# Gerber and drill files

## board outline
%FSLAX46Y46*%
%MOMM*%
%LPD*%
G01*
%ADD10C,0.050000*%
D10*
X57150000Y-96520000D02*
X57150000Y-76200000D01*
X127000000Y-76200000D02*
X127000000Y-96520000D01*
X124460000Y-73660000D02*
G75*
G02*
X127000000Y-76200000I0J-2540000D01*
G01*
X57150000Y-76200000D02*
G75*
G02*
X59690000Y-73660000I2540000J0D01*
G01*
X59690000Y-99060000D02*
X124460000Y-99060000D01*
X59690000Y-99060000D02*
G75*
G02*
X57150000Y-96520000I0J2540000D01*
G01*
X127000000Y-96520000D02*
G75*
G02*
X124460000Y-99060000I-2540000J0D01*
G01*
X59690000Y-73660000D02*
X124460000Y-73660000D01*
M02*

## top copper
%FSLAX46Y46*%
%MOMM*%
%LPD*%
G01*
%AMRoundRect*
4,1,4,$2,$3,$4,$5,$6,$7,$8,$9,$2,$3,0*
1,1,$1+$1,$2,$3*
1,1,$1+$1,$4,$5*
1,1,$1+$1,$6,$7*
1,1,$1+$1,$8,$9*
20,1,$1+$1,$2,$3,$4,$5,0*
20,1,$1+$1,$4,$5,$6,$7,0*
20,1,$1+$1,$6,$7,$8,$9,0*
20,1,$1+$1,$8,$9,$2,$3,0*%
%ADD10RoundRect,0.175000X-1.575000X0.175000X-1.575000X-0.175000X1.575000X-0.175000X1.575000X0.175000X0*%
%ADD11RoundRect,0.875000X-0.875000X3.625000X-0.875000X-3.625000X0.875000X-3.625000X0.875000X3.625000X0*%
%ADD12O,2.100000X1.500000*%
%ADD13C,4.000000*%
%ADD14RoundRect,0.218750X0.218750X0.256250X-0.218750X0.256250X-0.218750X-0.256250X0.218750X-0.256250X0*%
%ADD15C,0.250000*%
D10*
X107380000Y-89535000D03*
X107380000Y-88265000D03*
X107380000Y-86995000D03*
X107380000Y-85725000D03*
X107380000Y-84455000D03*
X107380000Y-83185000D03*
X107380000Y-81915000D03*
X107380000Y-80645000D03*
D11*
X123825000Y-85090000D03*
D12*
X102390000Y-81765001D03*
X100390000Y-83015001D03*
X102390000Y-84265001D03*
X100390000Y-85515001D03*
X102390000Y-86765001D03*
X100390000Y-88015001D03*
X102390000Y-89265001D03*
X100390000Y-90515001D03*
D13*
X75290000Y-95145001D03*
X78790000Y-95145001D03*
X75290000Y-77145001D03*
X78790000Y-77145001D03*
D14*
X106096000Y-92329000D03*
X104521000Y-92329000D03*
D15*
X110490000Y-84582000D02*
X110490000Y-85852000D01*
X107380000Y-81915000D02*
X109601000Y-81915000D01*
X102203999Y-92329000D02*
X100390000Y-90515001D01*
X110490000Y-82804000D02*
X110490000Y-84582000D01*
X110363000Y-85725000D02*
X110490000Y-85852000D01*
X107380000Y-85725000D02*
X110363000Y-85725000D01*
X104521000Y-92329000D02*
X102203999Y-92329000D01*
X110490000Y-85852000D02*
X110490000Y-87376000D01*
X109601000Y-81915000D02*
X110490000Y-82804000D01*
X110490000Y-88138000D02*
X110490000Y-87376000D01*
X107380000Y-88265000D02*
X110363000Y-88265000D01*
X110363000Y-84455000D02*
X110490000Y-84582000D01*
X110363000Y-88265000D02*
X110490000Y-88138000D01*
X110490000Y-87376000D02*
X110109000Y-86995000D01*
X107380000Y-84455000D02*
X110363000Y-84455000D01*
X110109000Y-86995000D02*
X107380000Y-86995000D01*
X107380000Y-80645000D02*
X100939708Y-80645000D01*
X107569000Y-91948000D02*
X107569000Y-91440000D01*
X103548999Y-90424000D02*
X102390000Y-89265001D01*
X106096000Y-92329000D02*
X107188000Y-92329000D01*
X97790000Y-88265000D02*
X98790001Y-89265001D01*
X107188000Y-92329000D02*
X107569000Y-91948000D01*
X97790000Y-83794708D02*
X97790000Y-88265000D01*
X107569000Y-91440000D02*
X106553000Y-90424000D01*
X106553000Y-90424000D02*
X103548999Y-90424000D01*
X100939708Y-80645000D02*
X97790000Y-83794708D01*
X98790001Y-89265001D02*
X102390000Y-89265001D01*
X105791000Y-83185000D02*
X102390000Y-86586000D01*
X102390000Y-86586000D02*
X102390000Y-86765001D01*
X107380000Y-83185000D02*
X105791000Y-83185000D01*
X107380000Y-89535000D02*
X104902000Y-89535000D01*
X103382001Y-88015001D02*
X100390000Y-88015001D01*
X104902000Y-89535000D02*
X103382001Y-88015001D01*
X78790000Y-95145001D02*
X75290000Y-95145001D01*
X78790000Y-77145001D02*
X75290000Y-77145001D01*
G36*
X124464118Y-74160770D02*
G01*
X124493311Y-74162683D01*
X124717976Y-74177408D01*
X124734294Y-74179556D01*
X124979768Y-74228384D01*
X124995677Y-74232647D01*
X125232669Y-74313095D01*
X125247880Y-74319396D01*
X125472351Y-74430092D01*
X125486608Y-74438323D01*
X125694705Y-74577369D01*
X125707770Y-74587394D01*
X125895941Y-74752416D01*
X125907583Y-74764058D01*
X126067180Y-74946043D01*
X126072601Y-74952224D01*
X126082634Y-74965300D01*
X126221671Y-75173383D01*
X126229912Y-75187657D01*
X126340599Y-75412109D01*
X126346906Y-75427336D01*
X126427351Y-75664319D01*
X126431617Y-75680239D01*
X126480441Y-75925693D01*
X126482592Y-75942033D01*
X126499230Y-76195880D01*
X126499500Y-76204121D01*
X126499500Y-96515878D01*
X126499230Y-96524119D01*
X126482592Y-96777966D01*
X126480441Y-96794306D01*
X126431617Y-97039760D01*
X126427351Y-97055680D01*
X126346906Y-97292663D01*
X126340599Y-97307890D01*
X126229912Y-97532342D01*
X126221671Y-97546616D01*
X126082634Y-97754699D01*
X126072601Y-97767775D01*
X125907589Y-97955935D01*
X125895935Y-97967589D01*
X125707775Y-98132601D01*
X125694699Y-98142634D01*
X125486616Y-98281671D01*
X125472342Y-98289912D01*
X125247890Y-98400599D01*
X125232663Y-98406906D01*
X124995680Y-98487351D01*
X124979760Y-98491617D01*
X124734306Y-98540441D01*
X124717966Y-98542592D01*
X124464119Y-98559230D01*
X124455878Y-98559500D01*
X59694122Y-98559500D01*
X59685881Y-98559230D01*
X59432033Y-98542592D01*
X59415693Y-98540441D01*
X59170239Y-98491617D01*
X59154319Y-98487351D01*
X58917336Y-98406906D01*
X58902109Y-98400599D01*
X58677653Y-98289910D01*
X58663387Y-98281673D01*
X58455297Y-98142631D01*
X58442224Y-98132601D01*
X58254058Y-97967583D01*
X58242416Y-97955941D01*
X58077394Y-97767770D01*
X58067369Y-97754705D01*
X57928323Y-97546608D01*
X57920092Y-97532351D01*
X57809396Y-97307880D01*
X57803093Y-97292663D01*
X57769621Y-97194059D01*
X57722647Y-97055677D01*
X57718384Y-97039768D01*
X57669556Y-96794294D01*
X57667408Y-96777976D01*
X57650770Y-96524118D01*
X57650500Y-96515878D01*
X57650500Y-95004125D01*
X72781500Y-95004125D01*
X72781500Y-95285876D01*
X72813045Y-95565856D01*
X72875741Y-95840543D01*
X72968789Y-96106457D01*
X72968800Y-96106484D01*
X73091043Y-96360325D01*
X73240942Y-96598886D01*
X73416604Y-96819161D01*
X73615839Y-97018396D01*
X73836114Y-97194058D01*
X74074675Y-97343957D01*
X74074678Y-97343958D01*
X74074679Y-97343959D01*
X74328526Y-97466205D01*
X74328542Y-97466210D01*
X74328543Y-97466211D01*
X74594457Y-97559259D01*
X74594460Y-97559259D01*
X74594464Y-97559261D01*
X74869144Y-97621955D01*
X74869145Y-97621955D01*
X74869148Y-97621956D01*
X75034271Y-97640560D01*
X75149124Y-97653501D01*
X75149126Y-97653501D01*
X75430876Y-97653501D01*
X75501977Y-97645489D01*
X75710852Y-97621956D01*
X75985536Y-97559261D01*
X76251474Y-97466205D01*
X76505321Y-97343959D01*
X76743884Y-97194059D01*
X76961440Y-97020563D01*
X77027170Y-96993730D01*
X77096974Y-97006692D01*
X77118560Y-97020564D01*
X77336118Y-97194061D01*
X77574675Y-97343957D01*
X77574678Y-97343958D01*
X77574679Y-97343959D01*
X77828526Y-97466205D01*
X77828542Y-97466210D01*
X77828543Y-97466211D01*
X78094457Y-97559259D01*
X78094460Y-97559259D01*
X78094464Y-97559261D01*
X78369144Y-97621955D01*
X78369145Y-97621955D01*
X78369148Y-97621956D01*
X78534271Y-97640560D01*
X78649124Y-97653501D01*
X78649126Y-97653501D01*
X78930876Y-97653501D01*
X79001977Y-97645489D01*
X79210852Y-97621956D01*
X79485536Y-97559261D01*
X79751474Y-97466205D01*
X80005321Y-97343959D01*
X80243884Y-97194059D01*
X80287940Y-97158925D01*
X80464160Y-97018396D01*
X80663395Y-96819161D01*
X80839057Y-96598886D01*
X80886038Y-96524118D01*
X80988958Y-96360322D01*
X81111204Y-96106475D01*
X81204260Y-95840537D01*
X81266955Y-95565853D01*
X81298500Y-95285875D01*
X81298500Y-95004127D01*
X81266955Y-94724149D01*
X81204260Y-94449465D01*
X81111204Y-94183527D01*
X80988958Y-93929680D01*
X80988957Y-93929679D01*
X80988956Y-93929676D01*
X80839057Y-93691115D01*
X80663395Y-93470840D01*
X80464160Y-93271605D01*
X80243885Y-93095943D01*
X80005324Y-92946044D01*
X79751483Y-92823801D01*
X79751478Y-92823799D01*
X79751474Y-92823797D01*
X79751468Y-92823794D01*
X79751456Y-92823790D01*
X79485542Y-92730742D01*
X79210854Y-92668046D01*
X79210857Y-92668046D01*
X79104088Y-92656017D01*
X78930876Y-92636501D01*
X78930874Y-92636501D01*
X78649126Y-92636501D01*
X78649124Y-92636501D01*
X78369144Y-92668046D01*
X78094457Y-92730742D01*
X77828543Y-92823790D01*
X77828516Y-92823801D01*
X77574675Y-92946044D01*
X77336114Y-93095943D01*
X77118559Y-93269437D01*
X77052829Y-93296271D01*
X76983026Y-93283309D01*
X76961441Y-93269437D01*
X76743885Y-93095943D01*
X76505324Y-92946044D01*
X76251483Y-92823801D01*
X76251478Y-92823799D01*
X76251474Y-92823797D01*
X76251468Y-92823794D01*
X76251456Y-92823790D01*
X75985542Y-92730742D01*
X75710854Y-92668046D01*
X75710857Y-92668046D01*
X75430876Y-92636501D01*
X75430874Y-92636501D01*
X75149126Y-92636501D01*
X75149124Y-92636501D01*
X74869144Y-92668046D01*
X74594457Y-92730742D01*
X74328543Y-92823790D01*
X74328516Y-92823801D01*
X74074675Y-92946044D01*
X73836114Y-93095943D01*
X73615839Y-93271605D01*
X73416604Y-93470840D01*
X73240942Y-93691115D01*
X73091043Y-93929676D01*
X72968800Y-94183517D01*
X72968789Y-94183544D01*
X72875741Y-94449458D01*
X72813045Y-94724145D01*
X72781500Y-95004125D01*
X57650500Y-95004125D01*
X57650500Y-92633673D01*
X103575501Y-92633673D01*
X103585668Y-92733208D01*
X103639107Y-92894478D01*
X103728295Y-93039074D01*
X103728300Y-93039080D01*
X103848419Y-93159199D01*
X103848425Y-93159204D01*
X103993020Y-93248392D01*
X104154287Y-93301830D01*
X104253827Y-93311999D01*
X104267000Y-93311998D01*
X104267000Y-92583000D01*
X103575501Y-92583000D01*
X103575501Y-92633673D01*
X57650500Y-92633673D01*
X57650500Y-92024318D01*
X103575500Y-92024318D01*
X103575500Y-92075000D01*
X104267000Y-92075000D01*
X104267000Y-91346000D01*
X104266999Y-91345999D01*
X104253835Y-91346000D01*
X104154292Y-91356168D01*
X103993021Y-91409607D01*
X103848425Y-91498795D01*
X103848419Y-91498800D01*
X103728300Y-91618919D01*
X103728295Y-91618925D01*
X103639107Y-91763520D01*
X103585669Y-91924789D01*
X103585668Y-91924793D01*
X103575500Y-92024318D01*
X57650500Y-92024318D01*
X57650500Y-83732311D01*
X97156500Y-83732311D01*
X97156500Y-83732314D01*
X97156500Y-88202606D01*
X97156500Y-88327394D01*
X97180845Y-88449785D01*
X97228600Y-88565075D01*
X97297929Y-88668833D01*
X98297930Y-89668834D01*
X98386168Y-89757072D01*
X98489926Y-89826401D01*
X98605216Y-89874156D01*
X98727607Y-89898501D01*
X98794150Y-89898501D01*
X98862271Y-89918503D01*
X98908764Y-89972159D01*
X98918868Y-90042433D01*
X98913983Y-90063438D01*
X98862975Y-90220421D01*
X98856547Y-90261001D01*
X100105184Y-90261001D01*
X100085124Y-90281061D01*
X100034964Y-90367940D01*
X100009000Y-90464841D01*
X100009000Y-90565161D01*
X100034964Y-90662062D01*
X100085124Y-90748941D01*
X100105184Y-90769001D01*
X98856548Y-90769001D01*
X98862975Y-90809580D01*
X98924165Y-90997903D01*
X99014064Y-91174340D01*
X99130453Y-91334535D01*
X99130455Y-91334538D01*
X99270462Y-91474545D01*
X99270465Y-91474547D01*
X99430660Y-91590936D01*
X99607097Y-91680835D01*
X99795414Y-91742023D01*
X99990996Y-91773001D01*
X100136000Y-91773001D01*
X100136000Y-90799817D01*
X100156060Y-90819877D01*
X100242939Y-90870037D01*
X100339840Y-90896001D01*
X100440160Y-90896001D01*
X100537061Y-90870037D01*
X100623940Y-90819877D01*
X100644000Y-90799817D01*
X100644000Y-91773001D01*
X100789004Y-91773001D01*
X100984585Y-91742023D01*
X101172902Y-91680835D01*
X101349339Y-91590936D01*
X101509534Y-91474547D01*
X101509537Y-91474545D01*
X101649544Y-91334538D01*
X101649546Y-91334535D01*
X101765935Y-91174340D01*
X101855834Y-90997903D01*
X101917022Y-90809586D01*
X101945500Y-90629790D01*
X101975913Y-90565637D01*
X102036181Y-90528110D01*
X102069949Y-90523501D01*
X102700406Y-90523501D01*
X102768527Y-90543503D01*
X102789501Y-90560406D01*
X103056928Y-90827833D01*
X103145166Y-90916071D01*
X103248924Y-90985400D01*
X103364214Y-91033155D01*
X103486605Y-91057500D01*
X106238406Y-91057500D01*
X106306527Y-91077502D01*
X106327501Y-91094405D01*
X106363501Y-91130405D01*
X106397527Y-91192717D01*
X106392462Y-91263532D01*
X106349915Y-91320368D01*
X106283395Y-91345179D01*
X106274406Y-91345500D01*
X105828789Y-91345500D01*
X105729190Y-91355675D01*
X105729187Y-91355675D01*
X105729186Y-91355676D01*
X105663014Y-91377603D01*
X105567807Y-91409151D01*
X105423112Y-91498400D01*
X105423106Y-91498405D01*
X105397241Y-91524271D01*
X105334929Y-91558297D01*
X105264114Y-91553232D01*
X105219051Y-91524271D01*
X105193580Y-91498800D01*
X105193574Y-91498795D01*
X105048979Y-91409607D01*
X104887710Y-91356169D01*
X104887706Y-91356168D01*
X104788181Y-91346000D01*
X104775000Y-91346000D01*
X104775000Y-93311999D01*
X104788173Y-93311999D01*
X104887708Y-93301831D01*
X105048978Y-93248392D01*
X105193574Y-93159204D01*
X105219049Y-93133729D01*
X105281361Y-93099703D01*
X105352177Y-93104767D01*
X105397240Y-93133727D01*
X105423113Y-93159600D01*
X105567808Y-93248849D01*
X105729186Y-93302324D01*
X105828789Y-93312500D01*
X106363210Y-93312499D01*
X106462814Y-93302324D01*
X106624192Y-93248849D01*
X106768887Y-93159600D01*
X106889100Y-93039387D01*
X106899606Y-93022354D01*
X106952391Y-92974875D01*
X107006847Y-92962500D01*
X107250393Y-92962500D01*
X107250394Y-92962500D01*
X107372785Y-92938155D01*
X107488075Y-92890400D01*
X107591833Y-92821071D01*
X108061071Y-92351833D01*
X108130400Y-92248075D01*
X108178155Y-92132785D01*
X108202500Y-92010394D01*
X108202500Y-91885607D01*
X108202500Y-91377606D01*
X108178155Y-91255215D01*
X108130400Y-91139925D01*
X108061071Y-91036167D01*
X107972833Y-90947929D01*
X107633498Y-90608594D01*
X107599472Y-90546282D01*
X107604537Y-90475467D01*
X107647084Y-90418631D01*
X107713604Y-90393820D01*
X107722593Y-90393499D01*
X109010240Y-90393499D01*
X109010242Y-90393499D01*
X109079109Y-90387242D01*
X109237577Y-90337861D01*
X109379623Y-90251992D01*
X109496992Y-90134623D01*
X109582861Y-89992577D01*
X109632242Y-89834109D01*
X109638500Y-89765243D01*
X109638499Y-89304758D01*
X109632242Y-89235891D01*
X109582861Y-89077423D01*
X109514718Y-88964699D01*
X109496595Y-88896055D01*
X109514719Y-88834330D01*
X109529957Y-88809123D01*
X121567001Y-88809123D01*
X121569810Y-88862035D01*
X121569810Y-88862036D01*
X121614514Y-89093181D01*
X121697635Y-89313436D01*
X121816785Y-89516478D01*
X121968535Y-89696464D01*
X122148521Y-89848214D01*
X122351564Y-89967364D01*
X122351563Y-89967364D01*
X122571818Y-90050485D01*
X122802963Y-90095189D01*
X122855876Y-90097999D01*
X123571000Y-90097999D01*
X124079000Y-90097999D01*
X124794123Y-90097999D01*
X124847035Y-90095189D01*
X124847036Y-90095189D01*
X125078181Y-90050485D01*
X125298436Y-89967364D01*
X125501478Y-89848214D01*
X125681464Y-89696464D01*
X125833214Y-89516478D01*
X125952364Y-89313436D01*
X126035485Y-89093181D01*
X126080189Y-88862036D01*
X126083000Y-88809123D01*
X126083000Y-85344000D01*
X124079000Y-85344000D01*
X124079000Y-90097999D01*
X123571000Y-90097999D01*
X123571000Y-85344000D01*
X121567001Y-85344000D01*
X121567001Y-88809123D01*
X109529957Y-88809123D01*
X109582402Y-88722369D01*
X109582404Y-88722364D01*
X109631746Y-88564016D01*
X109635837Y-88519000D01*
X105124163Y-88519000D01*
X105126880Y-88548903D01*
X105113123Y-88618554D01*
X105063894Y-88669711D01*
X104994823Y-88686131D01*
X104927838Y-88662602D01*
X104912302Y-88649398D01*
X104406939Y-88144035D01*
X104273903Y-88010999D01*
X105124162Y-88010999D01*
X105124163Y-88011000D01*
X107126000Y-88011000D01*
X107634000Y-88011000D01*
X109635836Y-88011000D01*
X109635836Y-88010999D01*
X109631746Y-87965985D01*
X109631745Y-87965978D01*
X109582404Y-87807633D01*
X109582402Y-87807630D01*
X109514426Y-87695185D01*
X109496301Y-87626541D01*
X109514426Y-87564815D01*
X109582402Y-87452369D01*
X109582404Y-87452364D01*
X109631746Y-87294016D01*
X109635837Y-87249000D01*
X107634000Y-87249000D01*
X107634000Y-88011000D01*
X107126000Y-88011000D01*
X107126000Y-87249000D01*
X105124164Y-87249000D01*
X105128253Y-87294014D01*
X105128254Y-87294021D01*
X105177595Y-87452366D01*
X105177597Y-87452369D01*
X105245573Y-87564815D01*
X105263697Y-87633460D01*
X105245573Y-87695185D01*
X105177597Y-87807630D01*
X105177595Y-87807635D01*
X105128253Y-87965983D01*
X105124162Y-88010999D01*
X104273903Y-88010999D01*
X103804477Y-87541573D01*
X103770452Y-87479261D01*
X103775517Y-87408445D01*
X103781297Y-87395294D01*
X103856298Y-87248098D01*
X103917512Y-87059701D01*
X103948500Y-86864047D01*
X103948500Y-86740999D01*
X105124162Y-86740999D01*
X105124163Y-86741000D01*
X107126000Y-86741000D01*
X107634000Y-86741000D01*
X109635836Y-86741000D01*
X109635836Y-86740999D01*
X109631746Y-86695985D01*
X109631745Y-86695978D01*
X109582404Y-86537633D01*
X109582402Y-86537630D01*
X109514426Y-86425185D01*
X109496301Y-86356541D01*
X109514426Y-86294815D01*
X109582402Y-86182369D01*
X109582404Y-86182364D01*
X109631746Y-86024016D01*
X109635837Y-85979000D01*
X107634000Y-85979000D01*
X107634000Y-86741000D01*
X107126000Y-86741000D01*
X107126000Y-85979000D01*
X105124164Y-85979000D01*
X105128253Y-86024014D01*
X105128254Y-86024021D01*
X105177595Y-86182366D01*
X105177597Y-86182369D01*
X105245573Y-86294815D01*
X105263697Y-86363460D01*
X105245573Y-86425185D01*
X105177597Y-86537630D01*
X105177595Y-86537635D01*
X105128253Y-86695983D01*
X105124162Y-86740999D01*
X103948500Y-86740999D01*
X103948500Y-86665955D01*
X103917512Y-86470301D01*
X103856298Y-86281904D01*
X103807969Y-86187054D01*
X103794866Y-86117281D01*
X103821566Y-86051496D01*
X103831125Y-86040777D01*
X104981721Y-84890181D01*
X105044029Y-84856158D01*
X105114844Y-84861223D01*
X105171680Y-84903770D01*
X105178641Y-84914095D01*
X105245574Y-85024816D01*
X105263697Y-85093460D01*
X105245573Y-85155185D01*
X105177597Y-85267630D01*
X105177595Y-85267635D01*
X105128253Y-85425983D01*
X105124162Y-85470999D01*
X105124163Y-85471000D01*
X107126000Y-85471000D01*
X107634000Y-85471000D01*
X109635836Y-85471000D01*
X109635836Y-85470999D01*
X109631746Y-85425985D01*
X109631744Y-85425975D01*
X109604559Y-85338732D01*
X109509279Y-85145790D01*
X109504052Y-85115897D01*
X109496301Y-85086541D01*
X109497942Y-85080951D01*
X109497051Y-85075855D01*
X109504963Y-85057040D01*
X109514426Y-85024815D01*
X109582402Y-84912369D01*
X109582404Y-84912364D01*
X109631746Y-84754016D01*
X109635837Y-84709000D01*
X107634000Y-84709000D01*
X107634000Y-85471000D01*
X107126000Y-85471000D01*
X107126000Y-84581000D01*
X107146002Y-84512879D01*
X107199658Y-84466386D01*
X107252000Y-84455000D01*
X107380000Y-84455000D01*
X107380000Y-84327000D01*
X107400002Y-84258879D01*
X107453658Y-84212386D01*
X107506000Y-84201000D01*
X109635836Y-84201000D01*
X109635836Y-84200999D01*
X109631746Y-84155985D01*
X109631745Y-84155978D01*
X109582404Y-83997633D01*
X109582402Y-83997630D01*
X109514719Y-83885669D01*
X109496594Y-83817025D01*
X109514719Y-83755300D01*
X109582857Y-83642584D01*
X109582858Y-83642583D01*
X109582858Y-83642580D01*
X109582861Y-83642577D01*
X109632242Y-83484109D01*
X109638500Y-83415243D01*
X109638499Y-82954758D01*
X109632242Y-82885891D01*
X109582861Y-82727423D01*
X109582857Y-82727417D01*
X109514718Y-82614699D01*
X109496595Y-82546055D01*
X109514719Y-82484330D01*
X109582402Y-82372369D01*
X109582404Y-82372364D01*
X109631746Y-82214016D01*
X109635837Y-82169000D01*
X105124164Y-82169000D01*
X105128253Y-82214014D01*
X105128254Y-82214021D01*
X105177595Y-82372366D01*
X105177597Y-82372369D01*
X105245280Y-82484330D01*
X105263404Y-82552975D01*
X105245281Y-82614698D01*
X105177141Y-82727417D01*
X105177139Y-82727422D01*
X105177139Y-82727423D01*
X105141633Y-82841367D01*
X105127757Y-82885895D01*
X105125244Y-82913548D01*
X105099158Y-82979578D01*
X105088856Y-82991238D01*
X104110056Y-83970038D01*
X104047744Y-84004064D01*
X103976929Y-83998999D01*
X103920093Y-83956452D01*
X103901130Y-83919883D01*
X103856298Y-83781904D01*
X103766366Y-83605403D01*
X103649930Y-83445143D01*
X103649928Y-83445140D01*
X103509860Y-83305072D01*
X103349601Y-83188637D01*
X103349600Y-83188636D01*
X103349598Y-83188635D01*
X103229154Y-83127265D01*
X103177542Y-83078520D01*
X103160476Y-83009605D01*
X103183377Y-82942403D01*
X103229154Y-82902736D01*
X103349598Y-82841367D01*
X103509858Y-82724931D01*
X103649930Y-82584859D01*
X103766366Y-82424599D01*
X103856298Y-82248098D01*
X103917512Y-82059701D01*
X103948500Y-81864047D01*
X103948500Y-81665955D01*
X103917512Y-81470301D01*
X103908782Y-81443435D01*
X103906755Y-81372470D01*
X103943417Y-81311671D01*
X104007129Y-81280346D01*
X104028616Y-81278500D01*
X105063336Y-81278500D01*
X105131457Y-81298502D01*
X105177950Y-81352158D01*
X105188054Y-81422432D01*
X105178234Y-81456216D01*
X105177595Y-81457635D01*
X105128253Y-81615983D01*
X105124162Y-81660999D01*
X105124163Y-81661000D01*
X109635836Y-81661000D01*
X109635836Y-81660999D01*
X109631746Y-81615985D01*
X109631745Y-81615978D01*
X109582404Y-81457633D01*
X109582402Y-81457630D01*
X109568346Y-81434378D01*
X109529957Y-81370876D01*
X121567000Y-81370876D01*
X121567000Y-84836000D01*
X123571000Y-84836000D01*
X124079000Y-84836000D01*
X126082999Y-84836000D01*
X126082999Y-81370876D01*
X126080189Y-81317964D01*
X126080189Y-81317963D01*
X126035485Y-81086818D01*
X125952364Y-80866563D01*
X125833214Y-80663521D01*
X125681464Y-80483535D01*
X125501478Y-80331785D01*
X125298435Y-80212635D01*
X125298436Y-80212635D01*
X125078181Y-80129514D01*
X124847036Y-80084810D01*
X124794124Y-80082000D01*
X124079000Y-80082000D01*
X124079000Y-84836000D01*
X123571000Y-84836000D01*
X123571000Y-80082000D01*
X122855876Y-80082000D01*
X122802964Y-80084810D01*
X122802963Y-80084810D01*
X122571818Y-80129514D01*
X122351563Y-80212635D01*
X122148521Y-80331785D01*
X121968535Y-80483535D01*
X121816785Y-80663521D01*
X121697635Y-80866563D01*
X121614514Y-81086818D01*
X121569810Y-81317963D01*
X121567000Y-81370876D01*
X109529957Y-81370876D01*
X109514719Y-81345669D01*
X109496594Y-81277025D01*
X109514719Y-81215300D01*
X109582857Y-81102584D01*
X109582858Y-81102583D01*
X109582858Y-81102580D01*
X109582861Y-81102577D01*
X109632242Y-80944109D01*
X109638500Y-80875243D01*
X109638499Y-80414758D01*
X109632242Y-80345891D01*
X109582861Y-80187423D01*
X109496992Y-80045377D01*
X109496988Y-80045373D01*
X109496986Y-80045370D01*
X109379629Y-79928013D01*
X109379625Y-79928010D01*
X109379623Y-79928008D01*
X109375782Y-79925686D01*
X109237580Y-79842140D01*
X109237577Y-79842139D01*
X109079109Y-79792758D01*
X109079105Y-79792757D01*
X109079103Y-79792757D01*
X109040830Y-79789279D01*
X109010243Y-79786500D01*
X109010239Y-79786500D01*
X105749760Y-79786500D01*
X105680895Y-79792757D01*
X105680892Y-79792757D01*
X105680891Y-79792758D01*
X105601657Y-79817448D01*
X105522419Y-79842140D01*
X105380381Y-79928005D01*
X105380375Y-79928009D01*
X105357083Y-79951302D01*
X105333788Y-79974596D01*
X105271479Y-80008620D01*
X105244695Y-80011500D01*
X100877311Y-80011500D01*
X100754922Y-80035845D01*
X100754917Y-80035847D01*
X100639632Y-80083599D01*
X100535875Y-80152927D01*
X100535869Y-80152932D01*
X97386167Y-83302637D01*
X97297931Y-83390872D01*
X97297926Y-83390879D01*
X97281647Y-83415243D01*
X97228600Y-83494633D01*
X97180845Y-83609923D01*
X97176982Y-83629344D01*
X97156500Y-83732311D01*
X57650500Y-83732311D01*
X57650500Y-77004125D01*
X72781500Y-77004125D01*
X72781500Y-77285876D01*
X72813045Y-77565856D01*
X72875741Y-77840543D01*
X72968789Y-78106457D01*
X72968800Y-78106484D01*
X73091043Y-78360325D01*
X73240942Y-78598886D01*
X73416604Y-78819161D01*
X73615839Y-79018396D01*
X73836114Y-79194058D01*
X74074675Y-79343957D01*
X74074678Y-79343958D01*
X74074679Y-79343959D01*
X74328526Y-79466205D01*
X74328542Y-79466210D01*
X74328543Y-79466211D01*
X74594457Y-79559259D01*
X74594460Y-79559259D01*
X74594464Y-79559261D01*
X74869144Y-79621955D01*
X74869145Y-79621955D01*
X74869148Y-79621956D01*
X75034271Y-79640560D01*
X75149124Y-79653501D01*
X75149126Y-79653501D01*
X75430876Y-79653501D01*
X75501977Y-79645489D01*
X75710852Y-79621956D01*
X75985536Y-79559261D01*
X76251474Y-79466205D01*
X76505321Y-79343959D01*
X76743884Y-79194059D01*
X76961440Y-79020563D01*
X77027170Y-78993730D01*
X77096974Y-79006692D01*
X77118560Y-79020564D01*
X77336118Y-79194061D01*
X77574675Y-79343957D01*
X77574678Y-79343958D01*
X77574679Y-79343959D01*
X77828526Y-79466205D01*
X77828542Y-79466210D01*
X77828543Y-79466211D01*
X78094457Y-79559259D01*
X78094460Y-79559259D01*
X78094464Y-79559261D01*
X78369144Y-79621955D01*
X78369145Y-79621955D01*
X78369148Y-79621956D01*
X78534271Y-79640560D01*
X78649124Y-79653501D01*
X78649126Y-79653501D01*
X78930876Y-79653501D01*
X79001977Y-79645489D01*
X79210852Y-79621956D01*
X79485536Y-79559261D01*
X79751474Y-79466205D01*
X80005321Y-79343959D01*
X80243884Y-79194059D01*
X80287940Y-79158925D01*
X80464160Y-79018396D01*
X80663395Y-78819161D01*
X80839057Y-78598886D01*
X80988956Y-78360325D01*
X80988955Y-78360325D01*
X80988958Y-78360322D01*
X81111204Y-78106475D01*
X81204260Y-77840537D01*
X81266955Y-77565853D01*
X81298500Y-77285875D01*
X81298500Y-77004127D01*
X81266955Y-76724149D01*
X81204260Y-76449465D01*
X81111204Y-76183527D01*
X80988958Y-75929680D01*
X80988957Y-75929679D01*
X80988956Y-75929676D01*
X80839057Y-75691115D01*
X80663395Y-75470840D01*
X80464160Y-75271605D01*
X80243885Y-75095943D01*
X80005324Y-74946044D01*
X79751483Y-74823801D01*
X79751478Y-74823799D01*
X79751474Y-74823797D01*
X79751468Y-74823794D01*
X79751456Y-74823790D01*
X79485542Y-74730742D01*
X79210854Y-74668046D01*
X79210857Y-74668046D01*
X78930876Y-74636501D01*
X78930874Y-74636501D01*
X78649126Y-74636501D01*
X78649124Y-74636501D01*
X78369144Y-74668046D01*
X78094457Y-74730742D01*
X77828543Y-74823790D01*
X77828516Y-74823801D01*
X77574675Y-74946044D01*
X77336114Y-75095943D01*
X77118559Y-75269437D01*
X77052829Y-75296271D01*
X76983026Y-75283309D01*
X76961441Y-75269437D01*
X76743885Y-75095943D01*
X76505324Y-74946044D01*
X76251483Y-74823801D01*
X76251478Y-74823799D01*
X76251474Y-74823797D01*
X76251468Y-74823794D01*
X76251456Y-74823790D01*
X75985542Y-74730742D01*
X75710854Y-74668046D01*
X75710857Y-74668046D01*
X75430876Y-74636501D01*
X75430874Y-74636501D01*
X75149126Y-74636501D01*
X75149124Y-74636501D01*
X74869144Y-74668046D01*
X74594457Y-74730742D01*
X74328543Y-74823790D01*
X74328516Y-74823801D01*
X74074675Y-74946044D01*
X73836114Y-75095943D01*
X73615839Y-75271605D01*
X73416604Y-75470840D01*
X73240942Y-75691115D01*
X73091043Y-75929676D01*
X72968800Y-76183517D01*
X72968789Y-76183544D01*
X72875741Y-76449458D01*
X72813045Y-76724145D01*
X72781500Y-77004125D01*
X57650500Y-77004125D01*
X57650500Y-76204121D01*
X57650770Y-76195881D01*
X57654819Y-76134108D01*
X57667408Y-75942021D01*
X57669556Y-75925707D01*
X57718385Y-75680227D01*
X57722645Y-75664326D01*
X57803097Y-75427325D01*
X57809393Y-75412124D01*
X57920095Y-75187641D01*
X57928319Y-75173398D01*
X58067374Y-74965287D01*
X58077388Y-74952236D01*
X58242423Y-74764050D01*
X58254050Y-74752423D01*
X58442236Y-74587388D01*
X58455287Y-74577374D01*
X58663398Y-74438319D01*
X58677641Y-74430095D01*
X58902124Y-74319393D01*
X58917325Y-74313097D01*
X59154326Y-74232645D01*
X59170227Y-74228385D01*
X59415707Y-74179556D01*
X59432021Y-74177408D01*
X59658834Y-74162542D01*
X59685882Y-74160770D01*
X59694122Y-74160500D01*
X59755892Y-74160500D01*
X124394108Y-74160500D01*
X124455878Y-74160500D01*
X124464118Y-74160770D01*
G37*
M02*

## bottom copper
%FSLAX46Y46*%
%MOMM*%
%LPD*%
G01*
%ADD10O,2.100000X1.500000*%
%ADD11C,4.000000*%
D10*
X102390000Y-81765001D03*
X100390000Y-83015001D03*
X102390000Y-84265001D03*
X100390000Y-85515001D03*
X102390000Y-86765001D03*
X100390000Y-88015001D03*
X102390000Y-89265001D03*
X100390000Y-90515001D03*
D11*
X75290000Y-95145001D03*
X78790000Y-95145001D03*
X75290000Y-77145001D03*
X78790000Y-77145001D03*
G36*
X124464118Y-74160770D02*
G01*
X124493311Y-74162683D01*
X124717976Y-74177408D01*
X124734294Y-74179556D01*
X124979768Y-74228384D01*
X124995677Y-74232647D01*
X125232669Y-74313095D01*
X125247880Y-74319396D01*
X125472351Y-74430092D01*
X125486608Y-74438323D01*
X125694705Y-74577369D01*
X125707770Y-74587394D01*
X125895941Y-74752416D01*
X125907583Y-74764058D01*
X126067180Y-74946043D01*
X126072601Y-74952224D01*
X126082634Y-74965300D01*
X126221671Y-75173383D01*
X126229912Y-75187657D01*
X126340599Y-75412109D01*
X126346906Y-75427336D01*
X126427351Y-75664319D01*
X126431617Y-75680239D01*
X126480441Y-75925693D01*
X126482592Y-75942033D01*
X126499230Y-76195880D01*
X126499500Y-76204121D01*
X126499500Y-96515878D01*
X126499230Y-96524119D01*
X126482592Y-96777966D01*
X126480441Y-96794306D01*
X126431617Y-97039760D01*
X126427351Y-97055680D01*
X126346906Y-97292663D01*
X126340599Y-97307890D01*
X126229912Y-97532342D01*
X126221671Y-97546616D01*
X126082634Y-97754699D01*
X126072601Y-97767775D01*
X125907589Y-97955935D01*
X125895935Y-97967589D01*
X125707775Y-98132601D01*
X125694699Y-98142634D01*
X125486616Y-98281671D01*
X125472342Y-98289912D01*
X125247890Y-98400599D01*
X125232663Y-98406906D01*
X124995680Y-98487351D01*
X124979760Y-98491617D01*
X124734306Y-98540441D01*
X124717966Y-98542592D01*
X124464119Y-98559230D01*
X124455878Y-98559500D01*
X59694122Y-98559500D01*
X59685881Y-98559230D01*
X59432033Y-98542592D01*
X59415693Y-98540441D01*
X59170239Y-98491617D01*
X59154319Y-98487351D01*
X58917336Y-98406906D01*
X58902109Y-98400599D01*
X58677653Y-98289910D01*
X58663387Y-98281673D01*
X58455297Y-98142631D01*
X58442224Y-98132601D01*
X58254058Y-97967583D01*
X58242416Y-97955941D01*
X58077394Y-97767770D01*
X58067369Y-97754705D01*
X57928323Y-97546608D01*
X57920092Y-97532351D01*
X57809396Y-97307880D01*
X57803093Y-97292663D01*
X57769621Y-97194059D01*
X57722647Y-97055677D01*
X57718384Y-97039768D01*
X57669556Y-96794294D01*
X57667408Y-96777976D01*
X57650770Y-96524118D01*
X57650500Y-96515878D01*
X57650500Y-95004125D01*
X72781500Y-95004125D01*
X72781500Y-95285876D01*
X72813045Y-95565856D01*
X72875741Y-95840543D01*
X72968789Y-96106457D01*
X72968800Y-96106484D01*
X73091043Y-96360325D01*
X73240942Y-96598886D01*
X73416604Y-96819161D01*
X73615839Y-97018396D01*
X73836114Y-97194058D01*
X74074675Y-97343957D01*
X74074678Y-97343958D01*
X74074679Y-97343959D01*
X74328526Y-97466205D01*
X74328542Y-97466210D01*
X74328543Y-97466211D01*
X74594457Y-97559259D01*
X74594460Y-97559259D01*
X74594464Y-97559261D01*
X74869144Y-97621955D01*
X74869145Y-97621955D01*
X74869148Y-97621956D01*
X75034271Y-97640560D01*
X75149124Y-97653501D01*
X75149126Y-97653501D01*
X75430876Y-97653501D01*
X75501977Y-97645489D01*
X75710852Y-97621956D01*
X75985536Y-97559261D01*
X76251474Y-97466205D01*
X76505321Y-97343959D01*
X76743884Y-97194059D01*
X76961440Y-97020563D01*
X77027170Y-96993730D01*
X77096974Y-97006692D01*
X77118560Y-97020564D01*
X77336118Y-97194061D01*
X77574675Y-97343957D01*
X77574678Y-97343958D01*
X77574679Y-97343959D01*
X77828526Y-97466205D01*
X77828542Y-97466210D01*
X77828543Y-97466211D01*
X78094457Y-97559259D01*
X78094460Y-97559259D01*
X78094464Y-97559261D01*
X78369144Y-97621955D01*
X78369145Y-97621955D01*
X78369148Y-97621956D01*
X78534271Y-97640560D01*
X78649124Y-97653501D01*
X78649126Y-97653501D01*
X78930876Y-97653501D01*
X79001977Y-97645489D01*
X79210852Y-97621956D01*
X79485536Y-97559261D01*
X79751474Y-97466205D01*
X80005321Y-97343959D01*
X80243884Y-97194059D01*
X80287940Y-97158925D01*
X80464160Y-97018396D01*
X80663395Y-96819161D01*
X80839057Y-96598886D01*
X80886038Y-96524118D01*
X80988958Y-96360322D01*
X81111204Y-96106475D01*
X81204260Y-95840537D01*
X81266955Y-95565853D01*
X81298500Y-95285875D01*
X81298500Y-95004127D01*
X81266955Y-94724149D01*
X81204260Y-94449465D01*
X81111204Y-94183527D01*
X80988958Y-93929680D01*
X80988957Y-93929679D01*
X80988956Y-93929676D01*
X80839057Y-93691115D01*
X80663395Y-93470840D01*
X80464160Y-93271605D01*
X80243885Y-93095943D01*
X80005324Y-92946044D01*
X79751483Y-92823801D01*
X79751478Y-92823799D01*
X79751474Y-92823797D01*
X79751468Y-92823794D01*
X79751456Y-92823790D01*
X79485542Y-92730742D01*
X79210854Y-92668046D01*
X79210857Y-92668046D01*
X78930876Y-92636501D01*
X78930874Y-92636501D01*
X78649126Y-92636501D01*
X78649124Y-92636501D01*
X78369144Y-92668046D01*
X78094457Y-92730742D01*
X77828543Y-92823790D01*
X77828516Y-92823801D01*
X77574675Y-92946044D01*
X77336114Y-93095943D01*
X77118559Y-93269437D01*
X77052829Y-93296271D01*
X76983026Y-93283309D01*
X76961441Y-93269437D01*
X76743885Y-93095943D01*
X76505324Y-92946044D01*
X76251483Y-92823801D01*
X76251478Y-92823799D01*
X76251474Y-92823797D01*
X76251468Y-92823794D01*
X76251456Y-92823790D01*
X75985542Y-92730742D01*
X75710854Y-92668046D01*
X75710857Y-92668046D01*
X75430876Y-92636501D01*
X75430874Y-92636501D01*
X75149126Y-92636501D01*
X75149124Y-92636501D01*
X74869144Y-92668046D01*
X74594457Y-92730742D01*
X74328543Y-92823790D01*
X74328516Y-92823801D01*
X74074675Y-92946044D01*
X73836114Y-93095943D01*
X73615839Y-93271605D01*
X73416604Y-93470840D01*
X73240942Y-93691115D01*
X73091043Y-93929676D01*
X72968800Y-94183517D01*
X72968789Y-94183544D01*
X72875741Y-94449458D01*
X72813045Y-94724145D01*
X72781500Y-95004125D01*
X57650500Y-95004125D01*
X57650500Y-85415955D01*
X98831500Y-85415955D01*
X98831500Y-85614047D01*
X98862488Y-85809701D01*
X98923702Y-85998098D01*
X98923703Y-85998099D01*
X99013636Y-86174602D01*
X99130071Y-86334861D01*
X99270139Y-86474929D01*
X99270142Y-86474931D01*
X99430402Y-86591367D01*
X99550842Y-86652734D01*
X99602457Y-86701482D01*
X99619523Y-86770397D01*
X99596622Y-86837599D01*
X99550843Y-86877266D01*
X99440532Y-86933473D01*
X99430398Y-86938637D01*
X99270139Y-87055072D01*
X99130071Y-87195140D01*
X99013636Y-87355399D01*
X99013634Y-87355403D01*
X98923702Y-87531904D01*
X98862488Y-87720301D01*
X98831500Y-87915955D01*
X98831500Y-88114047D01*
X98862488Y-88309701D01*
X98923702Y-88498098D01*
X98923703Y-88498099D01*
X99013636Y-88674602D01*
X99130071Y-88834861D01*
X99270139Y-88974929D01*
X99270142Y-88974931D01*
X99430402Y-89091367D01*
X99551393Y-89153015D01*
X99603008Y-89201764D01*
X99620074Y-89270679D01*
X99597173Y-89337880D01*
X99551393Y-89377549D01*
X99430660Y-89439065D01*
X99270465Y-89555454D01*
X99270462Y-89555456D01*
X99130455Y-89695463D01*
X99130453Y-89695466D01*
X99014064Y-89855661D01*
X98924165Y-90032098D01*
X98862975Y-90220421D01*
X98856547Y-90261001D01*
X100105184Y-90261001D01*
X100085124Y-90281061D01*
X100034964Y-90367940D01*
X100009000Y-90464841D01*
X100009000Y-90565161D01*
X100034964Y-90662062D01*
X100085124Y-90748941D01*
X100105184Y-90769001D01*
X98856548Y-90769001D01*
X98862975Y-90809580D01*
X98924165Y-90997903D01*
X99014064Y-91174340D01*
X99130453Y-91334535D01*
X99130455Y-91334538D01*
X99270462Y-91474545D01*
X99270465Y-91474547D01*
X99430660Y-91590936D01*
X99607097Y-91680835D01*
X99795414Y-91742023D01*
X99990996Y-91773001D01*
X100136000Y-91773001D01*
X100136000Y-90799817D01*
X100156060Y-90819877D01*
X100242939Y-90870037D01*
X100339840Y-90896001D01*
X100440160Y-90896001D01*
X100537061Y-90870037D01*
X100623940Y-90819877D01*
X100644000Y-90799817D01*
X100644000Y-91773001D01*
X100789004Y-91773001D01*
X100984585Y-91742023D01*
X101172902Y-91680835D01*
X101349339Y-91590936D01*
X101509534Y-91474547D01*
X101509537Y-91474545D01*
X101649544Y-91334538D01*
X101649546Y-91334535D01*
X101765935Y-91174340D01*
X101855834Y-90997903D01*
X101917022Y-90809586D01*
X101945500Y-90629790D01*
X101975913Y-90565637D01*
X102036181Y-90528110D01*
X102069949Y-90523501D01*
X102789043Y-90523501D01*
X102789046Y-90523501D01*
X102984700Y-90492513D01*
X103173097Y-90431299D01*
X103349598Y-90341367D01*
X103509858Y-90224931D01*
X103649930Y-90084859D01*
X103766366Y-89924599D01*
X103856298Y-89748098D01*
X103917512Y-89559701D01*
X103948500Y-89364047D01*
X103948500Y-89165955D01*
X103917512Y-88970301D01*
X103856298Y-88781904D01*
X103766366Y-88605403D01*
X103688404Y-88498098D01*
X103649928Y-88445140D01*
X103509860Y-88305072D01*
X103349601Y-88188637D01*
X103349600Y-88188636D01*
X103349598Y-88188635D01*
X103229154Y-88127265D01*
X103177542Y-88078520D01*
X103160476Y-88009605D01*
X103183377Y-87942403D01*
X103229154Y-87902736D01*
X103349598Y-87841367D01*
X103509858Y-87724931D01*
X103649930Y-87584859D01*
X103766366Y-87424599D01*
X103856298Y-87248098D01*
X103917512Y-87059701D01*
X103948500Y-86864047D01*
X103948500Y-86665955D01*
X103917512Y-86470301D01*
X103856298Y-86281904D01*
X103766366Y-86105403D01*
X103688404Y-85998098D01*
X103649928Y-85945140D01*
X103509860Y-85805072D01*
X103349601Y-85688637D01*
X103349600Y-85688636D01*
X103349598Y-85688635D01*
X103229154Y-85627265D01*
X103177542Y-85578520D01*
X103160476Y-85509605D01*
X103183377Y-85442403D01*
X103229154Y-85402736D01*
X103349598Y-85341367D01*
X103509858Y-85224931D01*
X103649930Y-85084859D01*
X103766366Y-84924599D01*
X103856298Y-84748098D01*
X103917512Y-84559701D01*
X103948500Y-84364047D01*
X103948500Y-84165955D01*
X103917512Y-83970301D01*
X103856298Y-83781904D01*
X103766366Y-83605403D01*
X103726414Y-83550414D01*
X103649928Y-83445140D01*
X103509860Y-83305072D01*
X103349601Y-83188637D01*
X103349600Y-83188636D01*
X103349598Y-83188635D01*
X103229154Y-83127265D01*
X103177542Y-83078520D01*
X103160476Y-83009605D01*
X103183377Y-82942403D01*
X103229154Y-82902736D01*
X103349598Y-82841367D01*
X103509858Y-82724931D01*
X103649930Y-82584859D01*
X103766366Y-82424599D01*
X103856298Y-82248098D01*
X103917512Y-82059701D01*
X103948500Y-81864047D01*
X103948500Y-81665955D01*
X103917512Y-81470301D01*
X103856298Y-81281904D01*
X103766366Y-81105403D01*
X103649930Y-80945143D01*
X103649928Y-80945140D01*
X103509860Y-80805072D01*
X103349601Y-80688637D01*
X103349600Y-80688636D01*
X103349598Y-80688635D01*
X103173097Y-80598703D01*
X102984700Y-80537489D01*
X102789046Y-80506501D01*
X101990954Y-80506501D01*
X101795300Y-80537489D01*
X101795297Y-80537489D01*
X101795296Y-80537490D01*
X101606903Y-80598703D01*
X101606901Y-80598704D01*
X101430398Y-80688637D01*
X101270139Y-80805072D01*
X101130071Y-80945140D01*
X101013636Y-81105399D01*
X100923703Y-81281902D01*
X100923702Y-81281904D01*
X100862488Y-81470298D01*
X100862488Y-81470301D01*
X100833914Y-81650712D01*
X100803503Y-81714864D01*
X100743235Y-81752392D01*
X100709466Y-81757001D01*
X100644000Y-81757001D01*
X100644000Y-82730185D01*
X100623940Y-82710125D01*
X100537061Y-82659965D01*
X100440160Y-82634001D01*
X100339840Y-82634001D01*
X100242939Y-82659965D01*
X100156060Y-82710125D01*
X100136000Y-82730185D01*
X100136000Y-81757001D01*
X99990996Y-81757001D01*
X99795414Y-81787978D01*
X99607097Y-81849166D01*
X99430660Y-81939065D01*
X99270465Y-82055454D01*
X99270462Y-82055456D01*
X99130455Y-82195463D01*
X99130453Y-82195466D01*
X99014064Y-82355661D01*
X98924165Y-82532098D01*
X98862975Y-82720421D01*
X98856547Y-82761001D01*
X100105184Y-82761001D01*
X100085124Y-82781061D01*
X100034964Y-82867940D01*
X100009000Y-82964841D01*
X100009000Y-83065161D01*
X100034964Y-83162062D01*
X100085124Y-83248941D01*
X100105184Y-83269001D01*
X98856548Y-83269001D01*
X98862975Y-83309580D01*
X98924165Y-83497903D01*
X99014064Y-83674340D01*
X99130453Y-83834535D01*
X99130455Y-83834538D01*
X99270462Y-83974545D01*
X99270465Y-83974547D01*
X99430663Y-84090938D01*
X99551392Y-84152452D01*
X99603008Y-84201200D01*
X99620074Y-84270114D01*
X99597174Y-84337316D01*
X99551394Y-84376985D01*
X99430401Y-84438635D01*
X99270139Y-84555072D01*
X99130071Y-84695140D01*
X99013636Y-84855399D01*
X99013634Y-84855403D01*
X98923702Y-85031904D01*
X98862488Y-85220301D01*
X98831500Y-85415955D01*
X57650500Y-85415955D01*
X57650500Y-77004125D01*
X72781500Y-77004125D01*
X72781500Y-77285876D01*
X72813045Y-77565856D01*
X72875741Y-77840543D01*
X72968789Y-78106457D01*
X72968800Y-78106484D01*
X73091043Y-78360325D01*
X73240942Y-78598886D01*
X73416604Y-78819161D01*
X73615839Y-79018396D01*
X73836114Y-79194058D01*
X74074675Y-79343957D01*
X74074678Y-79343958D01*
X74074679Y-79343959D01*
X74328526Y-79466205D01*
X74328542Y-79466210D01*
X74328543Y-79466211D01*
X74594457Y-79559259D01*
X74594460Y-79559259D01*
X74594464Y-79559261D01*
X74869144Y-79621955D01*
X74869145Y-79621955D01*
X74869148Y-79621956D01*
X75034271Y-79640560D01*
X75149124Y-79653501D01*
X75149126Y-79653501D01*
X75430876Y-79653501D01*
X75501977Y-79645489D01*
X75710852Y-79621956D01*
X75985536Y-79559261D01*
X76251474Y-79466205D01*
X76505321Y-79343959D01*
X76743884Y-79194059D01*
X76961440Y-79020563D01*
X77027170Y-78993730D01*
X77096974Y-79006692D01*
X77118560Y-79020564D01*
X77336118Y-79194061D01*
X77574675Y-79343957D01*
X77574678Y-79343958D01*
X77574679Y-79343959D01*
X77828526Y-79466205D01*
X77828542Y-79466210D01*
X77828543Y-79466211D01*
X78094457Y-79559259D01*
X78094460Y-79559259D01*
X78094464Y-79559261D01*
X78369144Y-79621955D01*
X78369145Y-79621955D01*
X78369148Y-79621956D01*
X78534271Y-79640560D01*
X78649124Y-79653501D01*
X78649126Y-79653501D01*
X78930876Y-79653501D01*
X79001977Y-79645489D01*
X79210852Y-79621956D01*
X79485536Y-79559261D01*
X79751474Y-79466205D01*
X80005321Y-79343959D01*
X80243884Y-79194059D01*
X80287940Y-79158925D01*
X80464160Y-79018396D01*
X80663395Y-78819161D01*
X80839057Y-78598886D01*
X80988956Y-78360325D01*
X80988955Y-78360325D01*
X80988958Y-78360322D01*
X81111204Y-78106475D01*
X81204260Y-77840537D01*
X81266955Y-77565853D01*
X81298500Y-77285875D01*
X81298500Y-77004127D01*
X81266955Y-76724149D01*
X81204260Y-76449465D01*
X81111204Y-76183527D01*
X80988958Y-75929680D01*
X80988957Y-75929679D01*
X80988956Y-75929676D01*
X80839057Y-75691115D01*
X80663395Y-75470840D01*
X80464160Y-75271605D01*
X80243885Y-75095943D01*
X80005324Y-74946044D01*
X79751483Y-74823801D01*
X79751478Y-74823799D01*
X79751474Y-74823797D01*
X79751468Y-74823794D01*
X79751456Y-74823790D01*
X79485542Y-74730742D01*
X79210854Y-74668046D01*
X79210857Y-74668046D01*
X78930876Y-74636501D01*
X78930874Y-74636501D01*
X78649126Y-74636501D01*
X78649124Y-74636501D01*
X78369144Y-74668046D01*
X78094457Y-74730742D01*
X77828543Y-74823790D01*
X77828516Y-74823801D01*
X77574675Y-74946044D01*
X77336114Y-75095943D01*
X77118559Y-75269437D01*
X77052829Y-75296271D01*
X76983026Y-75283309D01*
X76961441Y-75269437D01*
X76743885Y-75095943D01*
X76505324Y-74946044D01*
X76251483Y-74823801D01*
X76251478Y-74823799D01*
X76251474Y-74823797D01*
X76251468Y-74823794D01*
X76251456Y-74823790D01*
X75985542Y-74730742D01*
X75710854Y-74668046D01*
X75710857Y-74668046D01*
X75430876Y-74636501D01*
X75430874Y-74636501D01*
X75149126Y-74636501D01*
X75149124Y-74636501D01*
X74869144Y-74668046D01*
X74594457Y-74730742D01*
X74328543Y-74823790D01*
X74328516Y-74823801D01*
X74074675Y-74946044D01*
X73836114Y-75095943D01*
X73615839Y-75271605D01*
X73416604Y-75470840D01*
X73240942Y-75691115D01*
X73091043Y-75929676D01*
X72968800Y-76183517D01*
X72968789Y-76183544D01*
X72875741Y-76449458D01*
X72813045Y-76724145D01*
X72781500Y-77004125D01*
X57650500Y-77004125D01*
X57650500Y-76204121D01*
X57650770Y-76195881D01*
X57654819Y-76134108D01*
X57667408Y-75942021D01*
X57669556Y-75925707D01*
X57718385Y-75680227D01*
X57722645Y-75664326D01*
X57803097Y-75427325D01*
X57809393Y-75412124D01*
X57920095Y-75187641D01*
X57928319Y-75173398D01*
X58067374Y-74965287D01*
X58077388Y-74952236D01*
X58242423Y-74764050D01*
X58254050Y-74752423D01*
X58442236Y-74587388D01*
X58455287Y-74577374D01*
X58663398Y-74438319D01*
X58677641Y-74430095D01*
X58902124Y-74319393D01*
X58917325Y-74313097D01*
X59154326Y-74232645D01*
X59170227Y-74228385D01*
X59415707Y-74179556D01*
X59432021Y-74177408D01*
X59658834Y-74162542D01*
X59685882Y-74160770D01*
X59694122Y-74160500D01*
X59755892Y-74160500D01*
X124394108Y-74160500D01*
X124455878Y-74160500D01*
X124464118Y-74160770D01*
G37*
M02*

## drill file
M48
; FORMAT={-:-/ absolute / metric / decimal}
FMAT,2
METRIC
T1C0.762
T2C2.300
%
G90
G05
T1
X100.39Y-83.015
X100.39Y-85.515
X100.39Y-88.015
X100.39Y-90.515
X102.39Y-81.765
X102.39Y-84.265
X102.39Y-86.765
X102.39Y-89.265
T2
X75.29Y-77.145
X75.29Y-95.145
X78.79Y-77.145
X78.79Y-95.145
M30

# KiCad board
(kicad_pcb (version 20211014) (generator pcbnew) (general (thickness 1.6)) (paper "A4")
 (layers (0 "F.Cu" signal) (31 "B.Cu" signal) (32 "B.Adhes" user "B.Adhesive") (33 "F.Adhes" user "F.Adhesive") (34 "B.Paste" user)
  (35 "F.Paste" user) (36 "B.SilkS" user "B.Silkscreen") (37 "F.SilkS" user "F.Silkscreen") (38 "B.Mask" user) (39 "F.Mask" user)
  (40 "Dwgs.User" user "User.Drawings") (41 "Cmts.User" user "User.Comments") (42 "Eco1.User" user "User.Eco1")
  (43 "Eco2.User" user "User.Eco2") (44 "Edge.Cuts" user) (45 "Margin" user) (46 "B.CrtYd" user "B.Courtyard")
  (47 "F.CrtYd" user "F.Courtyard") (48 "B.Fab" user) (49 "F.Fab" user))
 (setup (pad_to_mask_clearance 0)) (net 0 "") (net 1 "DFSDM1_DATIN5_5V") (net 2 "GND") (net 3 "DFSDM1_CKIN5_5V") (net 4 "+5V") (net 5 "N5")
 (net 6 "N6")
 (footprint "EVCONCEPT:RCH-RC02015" (layer "F.Cu") (at 115.57 85.09 -90)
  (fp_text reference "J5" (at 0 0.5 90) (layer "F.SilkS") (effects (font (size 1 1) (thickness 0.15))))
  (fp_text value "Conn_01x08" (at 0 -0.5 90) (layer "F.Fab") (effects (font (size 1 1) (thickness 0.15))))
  (pad "1" smd roundrect locked (at 4.445 8.19 270) (size 0.7 3.5) (layers "F.Cu" "F.Paste" "F.Mask") (roundrect_rratio 0.25)
   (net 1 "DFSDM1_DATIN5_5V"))
  (pad "2" smd roundrect locked (at 3.175 8.19 270) (size 0.7 3.5) (layers "F.Cu" "F.Paste" "F.Mask") (roundrect_rratio 0.25) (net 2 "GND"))
  (pad "3" smd roundrect locked (at 1.905 8.19 270) (size 0.7 3.5) (layers "F.Cu" "F.Paste" "F.Mask") (roundrect_rratio 0.25) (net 2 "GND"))
  (pad "4" smd roundrect locked (at 0.635 8.19 270) (size 0.7 3.5) (layers "F.Cu" "F.Paste" "F.Mask") (roundrect_rratio 0.25) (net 2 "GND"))
  (pad "5" smd roundrect locked (at -0.635 8.19 270) (size 0.7 3.5) (layers "F.Cu" "F.Paste" "F.Mask") (roundrect_rratio 0.25) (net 2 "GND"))
  (pad "6" smd roundrect locked (at -1.905 8.19 270) (size 0.7 3.5) (layers "F.Cu" "F.Paste" "F.Mask") (roundrect_rratio 0.25)
   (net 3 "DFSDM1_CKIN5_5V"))
  (pad "7" smd roundrect locked (at -3.175 8.19 270) (size 0.7 3.5) (layers "F.Cu" "F.Paste" "F.Mask") (roundrect_rratio 0.25) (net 2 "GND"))
  (pad "8" smd roundrect locked (at -4.445 8.19 270) (size 0.7 3.5) (layers "F.Cu" "F.Paste" "F.Mask") (roundrect_rratio 0.25) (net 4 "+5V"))
  (pad "9" smd roundrect locked (at 0 -8.255 270) (size 9 3.5) (layers "F.Cu" "F.Paste" "F.Mask") (roundrect_rratio 0.25) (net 2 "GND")))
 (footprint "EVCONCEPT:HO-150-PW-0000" (layer "F.Cu") (at 100.39 86.145001)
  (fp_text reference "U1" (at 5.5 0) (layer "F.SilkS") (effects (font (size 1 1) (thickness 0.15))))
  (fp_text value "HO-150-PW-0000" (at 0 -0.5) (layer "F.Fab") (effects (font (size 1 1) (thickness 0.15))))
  (pad "1" thru_hole oval locked (at 2 -4.38) (size 2.1 1.5) (drill 0.762) (layers *.Cu *.Mask))
  (pad "2" thru_hole oval locked (at 0 -3.13) (size 2.1 1.5) (drill 0.762) (layers *.Cu *.Mask) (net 2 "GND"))
  (pad "3" thru_hole oval locked (at 2 -1.88) (size 2.1 1.5) (drill 0.762) (layers *.Cu *.Mask))
  (pad "4" thru_hole oval locked (at 0 -0.63) (size 2.1 1.5) (drill 0.762) (layers *.Cu *.Mask))
  (pad "5" thru_hole oval locked (at 2 0.62) (size 2.1 1.5) (drill 0.762) (layers *.Cu *.Mask) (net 3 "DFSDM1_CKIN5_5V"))
  (pad "6" thru_hole oval locked (at 0 1.87) (size 2.1 1.5) (drill 0.762) (layers *.Cu *.Mask) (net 1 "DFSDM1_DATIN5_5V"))
  (pad "7" thru_hole oval locked (at 2 3.12) (size 2.1 1.5) (drill 0.762) (layers *.Cu *.Mask) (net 4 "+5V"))
  (pad "8" thru_hole oval locked (at 0 4.37) (size 2.1 1.5) (drill 0.762) (layers *.Cu *.Mask) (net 2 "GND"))
  (pad "9" thru_hole circle locked (at -25.1 9) (size 4 4) (drill 2.3) (layers *.Cu *.Mask) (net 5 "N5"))
  (pad "9" thru_hole circle locked (at -21.6 9) (size 4 4) (drill 2.3) (layers *.Cu *.Mask) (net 5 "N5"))
  (pad "10" thru_hole circle locked (at -25.1 -9) (size 4 4) (drill 2.3) (layers *.Cu *.Mask) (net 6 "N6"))
  (pad "10" thru_hole circle locked (at -21.6 -9) (size 4 4) (drill 2.3) (layers *.Cu *.Mask) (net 6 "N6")))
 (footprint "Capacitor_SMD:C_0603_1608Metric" (layer "F.Cu") (at 105.3085 92.329 180)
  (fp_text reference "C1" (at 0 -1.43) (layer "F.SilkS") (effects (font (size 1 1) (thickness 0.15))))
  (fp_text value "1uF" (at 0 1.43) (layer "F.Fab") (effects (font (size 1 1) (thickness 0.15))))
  (pad "1" smd roundrect locked (at -0.7875 0 180) (size 0.875 0.95) (layers "F.Cu" "F.Paste" "F.Mask") (roundrect_rratio 0.25)
   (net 4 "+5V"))
  (pad "2" smd roundrect locked (at 0.7875 0 180) (size 0.875 0.95) (layers "F.Cu" "F.Paste" "F.Mask") (roundrect_rratio 0.25) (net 2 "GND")))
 (gr_line (start 57.15 96.52) (end 57.15 76.2) (layer "Edge.Cuts") (width 0.05))
 (gr_line (start 127 76.2) (end 127 96.52) (layer "Edge.Cuts") (width 0.05))
 (gr_arc (start 124.46 73.66) (mid 126.256051 74.403949) (end 127 76.2) (layer "Edge.Cuts") (width 0.05))
 (gr_arc (start 57.15 76.2) (mid 57.893949 74.403949) (end 59.69 73.66) (layer "Edge.Cuts") (width 0.05))
 (gr_line (start 59.69 99.06) (end 124.46 99.06) (layer "Edge.Cuts") (width 0.05))
 (gr_arc (start 59.69 99.06) (mid 57.893949 98.316051) (end 57.15 96.52) (layer "Edge.Cuts") (width 0.05))
 (gr_arc (start 127 96.52) (mid 126.256051 98.316051) (end 124.46 99.06) (layer "Edge.Cuts") (width 0.05))
 (gr_line (start 59.69 73.66) (end 124.46 73.66) (layer "Edge.Cuts") (width 0.05))
 (segment (start 110.49 84.582) (end 110.49 85.852) (width 0.25) (layer "F.Cu") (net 2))
 (segment (start 107.38 81.915) (end 109.601 81.915) (width 0.25) (layer "F.Cu") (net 2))
 (segment (start 102.203999 92.329) (end 100.39 90.515001) (width 0.25) (layer "F.Cu") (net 2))
 (segment (start 110.49 82.804) (end 110.49 84.582) (width 0.25) (layer "F.Cu") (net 2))
 (segment (start 110.363 85.725) (end 110.49 85.852) (width 0.25) (layer "F.Cu") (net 2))
 (segment (start 107.38 85.725) (end 110.363 85.725) (width 0.25) (layer "F.Cu") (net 2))
 (segment (start 104.521 92.329) (end 102.203999 92.329) (width 0.25) (layer "F.Cu") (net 2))
 (segment (start 110.49 85.852) (end 110.49 87.376) (width 0.25) (layer "F.Cu") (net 2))
 (segment (start 109.601 81.915) (end 110.49 82.804) (width 0.25) (layer "F.Cu") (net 2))
 (segment (start 110.49 88.138) (end 110.49 87.376) (width 0.25) (layer "F.Cu") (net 2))
 (segment (start 107.38 88.265) (end 110.363 88.265) (width 0.25) (layer "F.Cu") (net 2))
 (segment (start 110.363 84.455) (end 110.49 84.582) (width 0.25) (layer "F.Cu") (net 2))
 (segment (start 110.363 88.265) (end 110.49 88.138) (width 0.25) (layer "F.Cu") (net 2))
 (segment (start 110.49 87.376) (end 110.109 86.995) (width 0.25) (layer "F.Cu") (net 2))
 (segment (start 107.38 84.455) (end 110.363 84.455) (width 0.25) (layer "F.Cu") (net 2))
 (segment (start 110.109 86.995) (end 107.38 86.995) (width 0.25) (layer "F.Cu") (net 2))
 (segment (start 107.38 80.645) (end 100.939708 80.645) (width 0.25) (layer "F.Cu") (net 4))
 (segment (start 107.569 91.948) (end 107.569 91.44) (width 0.25) (layer "F.Cu") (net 4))
 (segment (start 103.548999 90.424) (end 102.39 89.265001) (width 0.25) (layer "F.Cu") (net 4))
 (segment (start 106.096 92.329) (end 107.188 92.329) (width 0.25) (layer "F.Cu") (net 4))
 (segment (start 97.79 88.265) (end 98.790001 89.265001) (width 0.25) (layer "F.Cu") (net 4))
 (segment (start 107.188 92.329) (end 107.569 91.948) (width 0.25) (layer "F.Cu") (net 4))
 (segment (start 97.79 83.794708) (end 97.79 88.265) (width 0.25) (layer "F.Cu") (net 4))
 (segment (start 107.569 91.44) (end 106.553 90.424) (width 0.25) (layer "F.Cu") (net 4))
 (segment (start 106.553 90.424) (end 103.548999 90.424) (width 0.25) (layer "F.Cu") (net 4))
 (segment (start 100.939708 80.645) (end 97.79 83.794708) (width 0.25) (layer "F.Cu") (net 4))
 (segment (start 98.790001 89.265001) (end 102.39 89.265001) (width 0.25) (layer "F.Cu") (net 4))
 (segment (start 105.791 83.185) (end 102.39 86.586) (width 0.25) (layer "F.Cu") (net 3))
 (segment (start 102.39 86.586) (end 102.39 86.765001) (width 0.25) (layer "F.Cu") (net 3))
 (segment (start 107.38 83.185) (end 105.791 83.185) (width 0.25) (layer "F.Cu") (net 3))
 (segment (start 107.38 89.535) (end 104.902 89.535) (width 0.25) (layer "F.Cu") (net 1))
 (segment (start 103.382001 88.015001) (end 100.39 88.015001) (width 0.25) (layer "F.Cu") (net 1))
 (segment (start 104.902 89.535) (end 103.382001 88.015001) (width 0.25) (layer "F.Cu") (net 1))
 (segment (start 78.79 95.145001) (end 75.29 95.145001) (width 0.25) (layer "F.Cu") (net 5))
 (segment (start 78.79 77.145001) (end 75.29 77.145001) (width 0.25) (layer "F.Cu") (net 6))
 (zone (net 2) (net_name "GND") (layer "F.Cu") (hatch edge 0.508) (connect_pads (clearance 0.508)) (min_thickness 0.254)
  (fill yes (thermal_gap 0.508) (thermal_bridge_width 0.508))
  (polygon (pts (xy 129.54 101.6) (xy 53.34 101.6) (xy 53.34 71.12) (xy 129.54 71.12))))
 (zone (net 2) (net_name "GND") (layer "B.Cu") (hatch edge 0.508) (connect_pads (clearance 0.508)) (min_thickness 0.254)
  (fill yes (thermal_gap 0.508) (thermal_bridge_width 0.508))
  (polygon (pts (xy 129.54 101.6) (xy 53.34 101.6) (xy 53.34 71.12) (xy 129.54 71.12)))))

